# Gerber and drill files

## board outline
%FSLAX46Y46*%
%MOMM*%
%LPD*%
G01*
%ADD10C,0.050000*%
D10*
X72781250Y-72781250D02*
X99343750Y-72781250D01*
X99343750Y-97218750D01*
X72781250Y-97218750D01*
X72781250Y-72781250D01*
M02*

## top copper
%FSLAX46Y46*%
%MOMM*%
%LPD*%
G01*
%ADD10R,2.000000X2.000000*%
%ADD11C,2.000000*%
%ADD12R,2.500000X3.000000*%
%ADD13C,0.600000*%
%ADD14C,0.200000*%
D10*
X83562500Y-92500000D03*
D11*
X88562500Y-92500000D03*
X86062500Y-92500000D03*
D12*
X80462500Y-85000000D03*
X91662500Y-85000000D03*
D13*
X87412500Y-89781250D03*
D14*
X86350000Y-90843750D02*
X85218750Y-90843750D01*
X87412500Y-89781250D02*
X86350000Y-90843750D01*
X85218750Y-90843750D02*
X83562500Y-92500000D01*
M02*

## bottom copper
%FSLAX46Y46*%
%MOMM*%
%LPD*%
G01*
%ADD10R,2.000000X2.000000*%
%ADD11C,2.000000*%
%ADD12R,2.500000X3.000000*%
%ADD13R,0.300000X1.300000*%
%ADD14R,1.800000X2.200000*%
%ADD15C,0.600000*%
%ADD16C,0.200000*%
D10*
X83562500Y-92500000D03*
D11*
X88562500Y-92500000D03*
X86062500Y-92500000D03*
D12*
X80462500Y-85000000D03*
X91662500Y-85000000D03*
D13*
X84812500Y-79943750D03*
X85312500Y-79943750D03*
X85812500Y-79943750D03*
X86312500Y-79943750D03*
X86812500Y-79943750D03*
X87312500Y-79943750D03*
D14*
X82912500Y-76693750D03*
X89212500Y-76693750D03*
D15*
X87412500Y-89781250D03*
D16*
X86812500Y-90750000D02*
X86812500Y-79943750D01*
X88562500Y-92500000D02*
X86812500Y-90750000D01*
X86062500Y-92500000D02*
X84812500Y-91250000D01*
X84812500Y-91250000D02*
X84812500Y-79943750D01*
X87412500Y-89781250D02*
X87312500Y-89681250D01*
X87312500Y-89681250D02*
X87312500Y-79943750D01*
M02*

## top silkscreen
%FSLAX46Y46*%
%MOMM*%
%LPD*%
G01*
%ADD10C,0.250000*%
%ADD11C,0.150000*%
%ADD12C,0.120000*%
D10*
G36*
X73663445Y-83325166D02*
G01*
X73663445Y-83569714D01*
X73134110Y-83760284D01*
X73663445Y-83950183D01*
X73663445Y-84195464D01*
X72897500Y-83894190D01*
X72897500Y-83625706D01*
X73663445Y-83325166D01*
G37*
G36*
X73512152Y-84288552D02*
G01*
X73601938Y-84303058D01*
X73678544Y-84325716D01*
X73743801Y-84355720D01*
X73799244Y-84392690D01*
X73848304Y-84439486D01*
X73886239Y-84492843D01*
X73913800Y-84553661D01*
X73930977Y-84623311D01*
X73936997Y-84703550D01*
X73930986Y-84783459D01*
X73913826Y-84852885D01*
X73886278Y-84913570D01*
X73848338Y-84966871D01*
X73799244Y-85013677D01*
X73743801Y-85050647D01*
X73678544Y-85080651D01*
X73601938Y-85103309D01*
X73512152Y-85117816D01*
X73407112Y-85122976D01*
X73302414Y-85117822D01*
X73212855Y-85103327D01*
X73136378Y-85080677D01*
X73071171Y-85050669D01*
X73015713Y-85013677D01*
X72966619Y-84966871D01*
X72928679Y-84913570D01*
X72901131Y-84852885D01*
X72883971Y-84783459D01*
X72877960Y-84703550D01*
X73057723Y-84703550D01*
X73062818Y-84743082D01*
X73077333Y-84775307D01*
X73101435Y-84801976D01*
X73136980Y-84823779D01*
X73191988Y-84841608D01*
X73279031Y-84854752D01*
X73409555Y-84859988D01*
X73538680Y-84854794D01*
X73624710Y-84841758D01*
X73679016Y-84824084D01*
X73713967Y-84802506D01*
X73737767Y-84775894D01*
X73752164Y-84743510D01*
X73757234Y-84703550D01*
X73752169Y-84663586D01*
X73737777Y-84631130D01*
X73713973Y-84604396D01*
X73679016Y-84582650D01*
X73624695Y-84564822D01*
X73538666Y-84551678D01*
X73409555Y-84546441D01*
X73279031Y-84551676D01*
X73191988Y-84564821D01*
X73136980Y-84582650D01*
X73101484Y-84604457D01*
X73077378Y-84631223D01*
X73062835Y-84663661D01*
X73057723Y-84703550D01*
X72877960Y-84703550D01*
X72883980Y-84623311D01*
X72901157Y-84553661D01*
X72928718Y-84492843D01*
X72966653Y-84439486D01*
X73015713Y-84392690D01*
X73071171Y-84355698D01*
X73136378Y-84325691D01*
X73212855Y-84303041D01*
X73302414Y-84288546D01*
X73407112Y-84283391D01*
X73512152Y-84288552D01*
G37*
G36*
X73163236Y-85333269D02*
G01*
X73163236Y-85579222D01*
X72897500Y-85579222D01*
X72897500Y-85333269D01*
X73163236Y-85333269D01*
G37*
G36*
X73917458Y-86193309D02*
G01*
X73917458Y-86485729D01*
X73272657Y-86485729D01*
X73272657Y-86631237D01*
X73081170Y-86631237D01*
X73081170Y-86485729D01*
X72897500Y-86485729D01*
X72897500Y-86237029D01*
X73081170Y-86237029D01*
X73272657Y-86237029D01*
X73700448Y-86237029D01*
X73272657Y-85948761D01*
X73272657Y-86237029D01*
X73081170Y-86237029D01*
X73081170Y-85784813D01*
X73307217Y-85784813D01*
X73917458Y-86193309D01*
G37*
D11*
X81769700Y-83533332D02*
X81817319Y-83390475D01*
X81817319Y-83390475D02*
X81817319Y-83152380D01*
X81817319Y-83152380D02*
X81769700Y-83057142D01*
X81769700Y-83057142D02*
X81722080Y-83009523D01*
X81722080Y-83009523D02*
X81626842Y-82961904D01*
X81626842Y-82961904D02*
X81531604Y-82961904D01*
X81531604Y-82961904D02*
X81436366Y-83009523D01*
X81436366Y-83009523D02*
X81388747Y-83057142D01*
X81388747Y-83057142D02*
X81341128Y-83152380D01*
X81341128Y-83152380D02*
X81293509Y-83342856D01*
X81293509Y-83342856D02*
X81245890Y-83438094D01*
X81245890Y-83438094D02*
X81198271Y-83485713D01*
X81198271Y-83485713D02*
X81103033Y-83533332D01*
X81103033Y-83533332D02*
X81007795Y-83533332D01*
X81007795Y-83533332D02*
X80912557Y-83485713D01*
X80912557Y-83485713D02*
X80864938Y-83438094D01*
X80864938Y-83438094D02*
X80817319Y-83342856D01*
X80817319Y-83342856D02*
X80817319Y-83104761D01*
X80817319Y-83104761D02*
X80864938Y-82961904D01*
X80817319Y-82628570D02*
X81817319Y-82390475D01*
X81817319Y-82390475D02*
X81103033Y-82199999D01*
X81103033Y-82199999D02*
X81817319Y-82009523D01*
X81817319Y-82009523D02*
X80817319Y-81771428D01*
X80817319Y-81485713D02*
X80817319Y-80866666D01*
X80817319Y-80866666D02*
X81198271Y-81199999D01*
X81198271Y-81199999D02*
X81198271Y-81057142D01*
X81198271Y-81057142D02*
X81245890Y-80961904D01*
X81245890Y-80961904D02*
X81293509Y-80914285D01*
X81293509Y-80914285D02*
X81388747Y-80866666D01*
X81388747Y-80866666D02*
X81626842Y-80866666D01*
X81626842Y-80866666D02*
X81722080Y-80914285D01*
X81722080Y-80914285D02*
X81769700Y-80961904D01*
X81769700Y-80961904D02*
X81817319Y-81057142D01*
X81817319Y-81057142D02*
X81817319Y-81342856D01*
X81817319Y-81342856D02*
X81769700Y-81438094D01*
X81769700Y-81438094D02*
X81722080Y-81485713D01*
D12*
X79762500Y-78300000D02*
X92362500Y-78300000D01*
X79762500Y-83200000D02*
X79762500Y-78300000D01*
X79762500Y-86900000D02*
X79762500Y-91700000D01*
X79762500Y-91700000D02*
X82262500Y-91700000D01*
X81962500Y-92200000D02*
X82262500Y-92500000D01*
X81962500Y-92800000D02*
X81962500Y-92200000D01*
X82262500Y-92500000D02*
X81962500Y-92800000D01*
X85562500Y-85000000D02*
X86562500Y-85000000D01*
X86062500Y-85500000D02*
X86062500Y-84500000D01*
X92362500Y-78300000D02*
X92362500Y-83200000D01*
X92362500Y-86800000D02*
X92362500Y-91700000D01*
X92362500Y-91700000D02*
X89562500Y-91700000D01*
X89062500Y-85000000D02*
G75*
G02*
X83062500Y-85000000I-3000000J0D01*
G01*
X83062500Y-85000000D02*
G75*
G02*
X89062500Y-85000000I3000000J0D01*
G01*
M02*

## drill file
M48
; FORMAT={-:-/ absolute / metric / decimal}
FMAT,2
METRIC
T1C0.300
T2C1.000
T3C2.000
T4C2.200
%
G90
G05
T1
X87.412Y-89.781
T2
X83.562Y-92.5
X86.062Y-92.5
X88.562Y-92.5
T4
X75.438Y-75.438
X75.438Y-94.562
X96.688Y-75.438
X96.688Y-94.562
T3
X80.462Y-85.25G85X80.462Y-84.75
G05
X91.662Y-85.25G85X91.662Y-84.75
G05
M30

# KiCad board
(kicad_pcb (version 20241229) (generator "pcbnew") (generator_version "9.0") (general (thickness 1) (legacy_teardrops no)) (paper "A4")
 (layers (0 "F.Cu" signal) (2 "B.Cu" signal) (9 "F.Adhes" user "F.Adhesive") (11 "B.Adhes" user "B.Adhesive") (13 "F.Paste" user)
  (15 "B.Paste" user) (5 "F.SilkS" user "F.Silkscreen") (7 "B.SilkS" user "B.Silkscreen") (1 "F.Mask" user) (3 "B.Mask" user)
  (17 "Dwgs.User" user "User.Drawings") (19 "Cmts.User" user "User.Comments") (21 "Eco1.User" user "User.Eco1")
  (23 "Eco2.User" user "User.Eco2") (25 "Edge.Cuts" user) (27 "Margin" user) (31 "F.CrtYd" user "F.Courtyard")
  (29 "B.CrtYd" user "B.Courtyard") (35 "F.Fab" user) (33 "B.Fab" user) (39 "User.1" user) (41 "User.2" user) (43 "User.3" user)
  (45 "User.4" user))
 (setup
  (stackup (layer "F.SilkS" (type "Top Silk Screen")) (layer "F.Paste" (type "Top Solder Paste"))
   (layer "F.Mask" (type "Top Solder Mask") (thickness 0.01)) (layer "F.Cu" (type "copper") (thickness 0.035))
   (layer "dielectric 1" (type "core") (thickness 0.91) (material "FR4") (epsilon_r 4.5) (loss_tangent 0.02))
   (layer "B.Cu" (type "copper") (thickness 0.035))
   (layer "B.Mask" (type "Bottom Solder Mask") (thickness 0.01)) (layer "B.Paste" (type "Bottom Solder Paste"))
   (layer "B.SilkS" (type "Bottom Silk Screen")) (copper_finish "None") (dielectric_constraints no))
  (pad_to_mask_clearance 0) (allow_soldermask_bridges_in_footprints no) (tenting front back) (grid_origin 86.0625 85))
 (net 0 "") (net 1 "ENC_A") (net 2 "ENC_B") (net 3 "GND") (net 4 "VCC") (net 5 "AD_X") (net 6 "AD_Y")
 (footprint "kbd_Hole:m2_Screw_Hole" (layer "F.Cu") (at 96.6875 75.4375)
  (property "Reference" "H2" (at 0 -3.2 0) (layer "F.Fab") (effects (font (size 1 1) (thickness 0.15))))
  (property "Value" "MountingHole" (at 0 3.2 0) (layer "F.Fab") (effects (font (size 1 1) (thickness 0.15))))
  (pad "" np_thru_hole circle (at 0 0) (size 2.2 2.2) (drill 2.2) (layers "*.Cu" "*.Mask")))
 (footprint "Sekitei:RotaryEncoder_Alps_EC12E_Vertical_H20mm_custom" (layer "F.Cu") (at 86.0625 85 90)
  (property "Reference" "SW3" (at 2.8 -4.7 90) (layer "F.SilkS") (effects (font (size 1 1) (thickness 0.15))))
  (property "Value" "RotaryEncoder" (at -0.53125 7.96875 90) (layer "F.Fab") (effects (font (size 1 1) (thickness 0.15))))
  (fp_line (start 6.7 -6.3) (end 6.7 6.3) (stroke (width 0.12) (type solid)) (layer "F.SilkS"))
  (fp_line (start 1.8 -6.3) (end 6.7 -6.3) (stroke (width 0.12) (type solid)) (layer "F.SilkS"))
  (fp_line (start -1.9 -6.3) (end -6.7 -6.3) (stroke (width 0.12) (type solid)) (layer "F.SilkS"))
  (fp_line (start -6.7 -6.3) (end -6.7 -3.8) (stroke (width 0.12) (type solid)) (layer "F.SilkS"))
  (fp_line (start -7.2 -4.1) (end -7.5 -3.8) (stroke (width 0.12) (type solid)) (layer "F.SilkS"))
  (fp_line (start -7.8 -4.1) (end -7.2 -4.1) (stroke (width 0.12) (type solid)) (layer "F.SilkS"))
  (fp_line (start -7.5 -3.8) (end -7.8 -4.1) (stroke (width 0.12) (type solid)) (layer "F.SilkS"))
  (fp_line (start 0 -0.5) (end 0 0.5) (stroke (width 0.12) (type solid)) (layer "F.SilkS"))
  (fp_line (start -0.5 0) (end 0.5 0) (stroke (width 0.12) (type solid)) (layer "F.SilkS"))
  (fp_line (start 6.7 6.3) (end 1.8 6.3) (stroke (width 0.12) (type solid)) (layer "F.SilkS"))
  (fp_line (start -1.8 6.3) (end -6.7 6.3) (stroke (width 0.12) (type solid)) (layer "F.SilkS"))
  (fp_line (start -6.7 6.3) (end -6.7 3.5) (stroke (width 0.12) (type solid)) (layer "F.SilkS"))
  (fp_circle (center 0 0) (end 3 0) (stroke (width 0.12) (type solid)) (fill no) (layer "F.SilkS"))
  (pad "A" thru_hole rect (at -7.5 -2.5 90) (size 2 2) (drill 1) (layers "*.Cu" "*.Mask") (remove_unused_layers no) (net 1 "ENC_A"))
  (pad "B" thru_hole circle (at -7.5 2.5 90) (size 2 2) (drill 1) (layers "*.Cu" "*.Mask") (remove_unused_layers no) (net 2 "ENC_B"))
  (pad "C" thru_hole circle (at -7.5 0 90) (size 2 2) (drill 1) (layers "*.Cu" "*.Mask") (remove_unused_layers no) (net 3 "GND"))
  (pad "MP" thru_hole rect (at 0 -5.6 90) (size 3 2.5) (drill oval 2.5 2) (layers "*.Cu" "*.Mask") (remove_unused_layers no))
  (pad "MP" thru_hole rect (at 0 5.6 90) (size 3 2.5) (drill oval 2.5 2) (layers "*.Cu" "*.Mask") (remove_unused_layers no)))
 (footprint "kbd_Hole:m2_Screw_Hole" (layer "F.Cu") (at 75.4375 94.5625)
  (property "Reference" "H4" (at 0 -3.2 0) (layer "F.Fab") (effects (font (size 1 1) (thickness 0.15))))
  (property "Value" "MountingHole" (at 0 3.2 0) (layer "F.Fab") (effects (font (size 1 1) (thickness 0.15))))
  (pad "" np_thru_hole circle (at 0 0) (size 2.2 2.2) (drill 2.2) (layers "*.Cu" "*.Mask")))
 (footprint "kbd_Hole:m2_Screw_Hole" (layer "F.Cu") (at 96.6875 94.5625)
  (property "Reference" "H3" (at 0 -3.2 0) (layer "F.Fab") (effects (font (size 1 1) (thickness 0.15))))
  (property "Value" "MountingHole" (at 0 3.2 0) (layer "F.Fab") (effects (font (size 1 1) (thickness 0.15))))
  (pad "" np_thru_hole circle (at 0 0) (size 2.2 2.2) (drill 2.2) (layers "*.Cu" "*.Mask")))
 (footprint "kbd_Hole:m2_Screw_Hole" (layer "F.Cu") (at 75.4375 75.4375)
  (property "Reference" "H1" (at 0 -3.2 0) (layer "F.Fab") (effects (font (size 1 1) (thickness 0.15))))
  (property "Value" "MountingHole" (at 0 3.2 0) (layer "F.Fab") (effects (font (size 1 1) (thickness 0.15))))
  (pad "" np_thru_hole circle (at 0 0) (size 2.2 2.2) (drill 2.2) (layers "*.Cu" "*.Mask")))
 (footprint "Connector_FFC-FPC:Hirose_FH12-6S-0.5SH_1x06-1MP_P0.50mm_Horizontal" (layer "B.Cu") (at 86.0625 78.09375)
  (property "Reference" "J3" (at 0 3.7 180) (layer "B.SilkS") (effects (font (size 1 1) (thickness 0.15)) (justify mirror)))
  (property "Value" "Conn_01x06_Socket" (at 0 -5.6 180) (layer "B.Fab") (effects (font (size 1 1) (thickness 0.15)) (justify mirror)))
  (pad "1" smd rect (at -1.25 1.85) (size 0.3 1.3) (layers "B.Cu" "B.Mask" "B.Paste") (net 3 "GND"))
  (pad "2" smd rect (at -0.75 1.85) (size 0.3 1.3) (layers "B.Cu" "B.Mask" "B.Paste") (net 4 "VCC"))
  (pad "3" smd rect (at -0.25 1.85) (size 0.3 1.3) (layers "B.Cu" "B.Mask" "B.Paste") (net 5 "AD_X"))
  (pad "4" smd rect (at 0.25 1.85) (size 0.3 1.3) (layers "B.Cu" "B.Mask" "B.Paste") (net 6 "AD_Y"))
  (pad "5" smd rect (at 0.75 1.85) (size 0.3 1.3) (layers "B.Cu" "B.Mask" "B.Paste") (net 2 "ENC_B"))
  (pad "6" smd rect (at 1.25 1.85) (size 0.3 1.3) (layers "B.Cu" "B.Mask" "B.Paste") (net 1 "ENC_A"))
  (pad "MP" smd rect (at -3.15 -1.4) (size 1.8 2.2) (layers "B.Cu" "B.Mask" "B.Paste"))
  (pad "MP" smd rect (at 3.15 -1.4) (size 1.8 2.2) (layers "B.Cu" "B.Mask" "B.Paste")))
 (gr_rect (start 72.78125 72.78125) (end 99.34375 97.21875) (stroke (width 0.05) (type default)) (fill no) (layer "Edge.Cuts"))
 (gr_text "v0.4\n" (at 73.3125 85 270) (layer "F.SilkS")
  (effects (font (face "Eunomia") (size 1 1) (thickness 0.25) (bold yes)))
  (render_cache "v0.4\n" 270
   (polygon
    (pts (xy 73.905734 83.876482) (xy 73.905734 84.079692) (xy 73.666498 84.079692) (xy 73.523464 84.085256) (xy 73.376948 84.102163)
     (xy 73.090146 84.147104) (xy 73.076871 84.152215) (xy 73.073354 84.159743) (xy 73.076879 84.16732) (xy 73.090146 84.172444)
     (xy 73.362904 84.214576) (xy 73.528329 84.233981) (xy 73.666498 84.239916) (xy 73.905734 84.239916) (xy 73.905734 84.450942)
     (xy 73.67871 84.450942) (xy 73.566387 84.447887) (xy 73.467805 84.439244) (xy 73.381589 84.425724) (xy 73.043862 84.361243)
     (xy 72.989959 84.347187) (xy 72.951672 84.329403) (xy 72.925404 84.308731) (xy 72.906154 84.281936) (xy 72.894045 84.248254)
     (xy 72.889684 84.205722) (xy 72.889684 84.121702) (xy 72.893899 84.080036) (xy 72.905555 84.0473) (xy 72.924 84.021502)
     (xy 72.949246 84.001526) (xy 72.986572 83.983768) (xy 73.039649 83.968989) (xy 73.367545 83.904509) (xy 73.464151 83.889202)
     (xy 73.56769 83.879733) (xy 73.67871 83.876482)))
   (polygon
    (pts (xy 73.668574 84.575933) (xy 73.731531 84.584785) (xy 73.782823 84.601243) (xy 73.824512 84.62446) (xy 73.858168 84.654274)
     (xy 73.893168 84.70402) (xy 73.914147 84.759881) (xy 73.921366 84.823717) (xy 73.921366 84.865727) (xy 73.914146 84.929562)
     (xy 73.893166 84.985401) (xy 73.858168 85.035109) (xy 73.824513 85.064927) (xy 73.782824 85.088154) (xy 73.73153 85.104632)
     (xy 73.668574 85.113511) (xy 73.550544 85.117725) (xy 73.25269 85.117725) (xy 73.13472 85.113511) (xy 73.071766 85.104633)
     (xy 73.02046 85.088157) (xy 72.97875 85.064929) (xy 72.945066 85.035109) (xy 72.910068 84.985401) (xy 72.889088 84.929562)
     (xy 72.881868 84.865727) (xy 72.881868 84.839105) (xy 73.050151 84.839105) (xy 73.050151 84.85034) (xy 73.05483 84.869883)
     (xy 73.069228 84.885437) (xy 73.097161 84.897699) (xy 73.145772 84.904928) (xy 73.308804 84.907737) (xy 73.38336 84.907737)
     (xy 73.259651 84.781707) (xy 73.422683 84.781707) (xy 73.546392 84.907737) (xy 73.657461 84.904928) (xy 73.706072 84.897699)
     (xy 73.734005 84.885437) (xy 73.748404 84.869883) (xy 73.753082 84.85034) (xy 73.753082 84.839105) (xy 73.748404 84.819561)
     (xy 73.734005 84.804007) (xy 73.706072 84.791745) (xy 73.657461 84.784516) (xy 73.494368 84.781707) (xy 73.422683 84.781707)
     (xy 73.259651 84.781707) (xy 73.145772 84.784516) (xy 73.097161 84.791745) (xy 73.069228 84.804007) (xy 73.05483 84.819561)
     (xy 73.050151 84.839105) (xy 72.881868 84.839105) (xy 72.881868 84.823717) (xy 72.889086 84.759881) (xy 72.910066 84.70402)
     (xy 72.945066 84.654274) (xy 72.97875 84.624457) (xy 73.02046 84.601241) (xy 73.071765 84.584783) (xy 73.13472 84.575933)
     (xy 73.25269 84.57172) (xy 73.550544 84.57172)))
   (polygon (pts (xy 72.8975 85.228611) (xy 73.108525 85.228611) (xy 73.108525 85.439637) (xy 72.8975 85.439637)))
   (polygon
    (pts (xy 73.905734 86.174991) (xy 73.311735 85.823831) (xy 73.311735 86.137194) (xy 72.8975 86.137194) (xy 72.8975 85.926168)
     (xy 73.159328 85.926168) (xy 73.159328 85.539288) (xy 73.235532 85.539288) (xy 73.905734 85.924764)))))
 (segment (start 86.8125 90.75) (end 86.8125 79.94375) (width 0.2) (layer "B.Cu") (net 2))
 (segment (start 88.5625 92.5) (end 86.8125 90.75) (width 0.2) (layer "B.Cu") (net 2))
 (segment (start 86.0625 92.5) (end 84.8125 91.25) (width 0.2) (layer "B.Cu") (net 3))
 (segment (start 84.8125 91.25) (end 84.8125 79.94375) (width 0.2) (layer "B.Cu") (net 3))
 (segment (start 86.35 90.84375) (end 85.21875 90.84375) (width 0.2) (layer "F.Cu") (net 1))
 (segment (start 87.4125 89.78125) (end 86.35 90.84375) (width 0.2) (layer "F.Cu") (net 1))
 (segment (start 85.21875 90.84375) (end 83.5625 92.5) (width 0.2) (layer "F.Cu") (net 1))
 (via (at 87.4125 89.78125) (size 0.6) (drill 0.3) (layers "F.Cu" "B.Cu") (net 1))
 (segment (start 87.4125 89.78125) (end 87.3125 89.68125) (width 0.2) (layer "B.Cu") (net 1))
 (segment (start 87.3125 89.68125) (end 87.3125 79.94375) (width 0.2) (layer "B.Cu") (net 1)))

